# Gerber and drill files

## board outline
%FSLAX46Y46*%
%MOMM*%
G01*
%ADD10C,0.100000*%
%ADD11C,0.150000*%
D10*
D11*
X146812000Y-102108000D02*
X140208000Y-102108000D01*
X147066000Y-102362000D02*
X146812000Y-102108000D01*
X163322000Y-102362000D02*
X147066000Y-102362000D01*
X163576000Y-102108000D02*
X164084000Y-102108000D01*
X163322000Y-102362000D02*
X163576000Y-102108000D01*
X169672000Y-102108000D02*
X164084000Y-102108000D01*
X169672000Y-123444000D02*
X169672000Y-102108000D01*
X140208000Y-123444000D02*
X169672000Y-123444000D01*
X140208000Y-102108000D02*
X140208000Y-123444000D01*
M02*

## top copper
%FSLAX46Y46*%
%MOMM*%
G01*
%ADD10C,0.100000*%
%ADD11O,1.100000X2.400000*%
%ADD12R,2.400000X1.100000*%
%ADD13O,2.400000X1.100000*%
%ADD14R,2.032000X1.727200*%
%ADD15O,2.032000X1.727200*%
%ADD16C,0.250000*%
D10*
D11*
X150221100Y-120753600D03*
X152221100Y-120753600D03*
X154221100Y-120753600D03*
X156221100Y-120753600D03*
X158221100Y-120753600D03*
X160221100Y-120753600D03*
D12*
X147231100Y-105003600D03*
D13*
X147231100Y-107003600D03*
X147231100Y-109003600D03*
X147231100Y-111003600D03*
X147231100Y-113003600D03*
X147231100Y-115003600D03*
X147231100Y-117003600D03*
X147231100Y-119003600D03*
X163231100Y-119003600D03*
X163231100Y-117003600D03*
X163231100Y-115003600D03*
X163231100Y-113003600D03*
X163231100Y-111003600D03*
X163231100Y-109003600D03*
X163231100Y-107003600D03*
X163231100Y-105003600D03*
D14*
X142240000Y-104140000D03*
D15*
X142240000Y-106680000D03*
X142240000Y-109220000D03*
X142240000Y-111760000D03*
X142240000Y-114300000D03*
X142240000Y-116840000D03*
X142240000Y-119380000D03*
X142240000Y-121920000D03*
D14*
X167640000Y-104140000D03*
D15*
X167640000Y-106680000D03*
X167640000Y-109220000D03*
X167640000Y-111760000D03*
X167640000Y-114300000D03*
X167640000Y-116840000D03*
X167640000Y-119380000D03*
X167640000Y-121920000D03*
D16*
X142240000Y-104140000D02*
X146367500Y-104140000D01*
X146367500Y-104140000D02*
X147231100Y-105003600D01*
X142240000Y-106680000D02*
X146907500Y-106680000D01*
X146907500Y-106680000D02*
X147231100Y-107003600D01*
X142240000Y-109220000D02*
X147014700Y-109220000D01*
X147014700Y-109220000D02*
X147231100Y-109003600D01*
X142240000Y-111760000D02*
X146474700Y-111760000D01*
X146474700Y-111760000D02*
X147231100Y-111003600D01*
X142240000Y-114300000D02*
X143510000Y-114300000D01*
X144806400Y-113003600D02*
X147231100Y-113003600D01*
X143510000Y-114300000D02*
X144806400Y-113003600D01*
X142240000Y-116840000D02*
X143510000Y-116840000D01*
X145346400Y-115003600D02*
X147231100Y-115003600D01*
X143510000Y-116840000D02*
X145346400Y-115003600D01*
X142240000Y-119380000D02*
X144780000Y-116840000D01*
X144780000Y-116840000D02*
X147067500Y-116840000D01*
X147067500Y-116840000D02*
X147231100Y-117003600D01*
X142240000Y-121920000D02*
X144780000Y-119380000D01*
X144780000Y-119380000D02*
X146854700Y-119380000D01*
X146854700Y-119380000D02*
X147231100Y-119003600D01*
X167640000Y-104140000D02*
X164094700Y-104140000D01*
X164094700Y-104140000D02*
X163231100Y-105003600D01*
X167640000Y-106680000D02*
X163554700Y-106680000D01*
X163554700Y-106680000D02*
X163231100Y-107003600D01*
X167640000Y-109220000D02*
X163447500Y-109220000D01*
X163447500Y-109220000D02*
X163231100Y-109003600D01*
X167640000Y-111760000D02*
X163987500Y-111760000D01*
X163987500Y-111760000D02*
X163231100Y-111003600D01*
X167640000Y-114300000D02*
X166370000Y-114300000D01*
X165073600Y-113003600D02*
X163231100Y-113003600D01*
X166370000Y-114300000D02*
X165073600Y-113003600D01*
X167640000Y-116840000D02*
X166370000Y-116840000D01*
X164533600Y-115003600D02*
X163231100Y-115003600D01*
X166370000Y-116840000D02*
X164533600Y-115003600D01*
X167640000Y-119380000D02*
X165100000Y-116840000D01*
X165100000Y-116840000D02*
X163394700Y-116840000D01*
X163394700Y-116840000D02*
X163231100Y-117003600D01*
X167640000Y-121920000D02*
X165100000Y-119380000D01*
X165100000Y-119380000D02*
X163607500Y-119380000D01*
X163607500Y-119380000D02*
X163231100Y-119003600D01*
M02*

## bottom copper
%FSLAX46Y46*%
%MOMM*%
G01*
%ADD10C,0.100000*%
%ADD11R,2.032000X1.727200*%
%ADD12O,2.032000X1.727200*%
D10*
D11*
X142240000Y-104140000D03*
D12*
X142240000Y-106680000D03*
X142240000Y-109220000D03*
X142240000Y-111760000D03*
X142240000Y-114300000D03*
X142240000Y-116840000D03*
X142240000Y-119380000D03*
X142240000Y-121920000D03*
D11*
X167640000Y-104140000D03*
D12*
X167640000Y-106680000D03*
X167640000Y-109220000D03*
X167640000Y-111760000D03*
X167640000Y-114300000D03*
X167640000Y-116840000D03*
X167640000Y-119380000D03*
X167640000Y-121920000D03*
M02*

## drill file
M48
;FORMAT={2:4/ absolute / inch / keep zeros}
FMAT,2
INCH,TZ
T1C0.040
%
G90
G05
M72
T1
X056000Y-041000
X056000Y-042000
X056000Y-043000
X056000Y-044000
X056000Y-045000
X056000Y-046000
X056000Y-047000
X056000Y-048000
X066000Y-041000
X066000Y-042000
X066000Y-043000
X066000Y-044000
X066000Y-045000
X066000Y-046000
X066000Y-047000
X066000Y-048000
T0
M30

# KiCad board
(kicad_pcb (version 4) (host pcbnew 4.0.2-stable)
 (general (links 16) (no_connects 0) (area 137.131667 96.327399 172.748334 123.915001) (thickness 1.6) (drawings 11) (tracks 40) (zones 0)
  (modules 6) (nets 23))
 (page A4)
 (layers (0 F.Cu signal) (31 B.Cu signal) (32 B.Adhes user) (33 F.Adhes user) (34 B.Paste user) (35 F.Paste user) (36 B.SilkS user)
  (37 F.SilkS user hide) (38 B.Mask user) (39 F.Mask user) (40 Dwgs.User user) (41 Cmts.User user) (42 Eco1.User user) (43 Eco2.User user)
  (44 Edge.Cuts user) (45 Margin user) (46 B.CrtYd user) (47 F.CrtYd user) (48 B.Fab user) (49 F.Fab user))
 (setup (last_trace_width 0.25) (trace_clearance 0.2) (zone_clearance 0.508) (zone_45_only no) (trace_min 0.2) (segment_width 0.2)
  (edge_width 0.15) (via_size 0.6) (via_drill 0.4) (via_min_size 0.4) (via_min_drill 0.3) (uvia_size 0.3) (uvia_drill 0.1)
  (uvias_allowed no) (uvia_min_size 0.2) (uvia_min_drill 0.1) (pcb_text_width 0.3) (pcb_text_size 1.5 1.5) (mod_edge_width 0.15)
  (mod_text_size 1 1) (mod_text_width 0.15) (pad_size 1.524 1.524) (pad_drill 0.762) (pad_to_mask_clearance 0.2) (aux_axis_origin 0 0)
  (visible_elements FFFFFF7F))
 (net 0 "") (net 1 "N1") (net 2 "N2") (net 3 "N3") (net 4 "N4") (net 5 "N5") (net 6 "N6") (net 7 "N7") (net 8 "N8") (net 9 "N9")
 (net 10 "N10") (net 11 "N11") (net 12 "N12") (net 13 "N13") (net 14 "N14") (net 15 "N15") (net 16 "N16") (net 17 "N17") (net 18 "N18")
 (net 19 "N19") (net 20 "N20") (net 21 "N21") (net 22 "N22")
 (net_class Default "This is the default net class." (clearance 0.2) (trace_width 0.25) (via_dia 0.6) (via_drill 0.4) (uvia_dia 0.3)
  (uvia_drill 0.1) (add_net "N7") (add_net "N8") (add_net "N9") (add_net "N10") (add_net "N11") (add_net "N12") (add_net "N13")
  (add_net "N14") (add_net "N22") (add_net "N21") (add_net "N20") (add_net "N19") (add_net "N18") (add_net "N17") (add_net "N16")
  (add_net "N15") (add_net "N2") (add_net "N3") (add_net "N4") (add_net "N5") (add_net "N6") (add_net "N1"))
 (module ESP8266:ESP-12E (layer F.Cu) (at 147.2311 105.0036)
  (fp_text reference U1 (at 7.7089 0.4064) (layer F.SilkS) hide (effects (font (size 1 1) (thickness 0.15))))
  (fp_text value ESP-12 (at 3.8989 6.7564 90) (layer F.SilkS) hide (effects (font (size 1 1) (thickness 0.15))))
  (pad 9 smd oval (at 2.99 15.75 90) (size 2.4 1.1) (layers F.Cu F.Paste F.Mask) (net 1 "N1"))
  (pad 10 smd oval (at 4.99 15.75 90) (size 2.4 1.1) (layers F.Cu F.Paste F.Mask) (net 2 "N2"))
  (pad 11 smd oval (at 6.99 15.75 90) (size 2.4 1.1) (layers F.Cu F.Paste F.Mask) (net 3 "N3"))
  (pad 12 smd oval (at 8.99 15.75 90) (size 2.4 1.1) (layers F.Cu F.Paste F.Mask) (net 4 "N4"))
  (pad 13 smd oval (at 10.99 15.75 90) (size 2.4 1.1) (layers F.Cu F.Paste F.Mask) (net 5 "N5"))
  (pad 14 smd oval (at 12.99 15.75 90) (size 2.4 1.1) (layers F.Cu F.Paste F.Mask) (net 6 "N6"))
  (pad 1 smd rect (at 0 0) (size 2.4 1.1) (layers F.Cu F.Paste F.Mask) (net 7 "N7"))
  (pad 2 smd oval (at 0 2) (size 2.4 1.1) (layers F.Cu F.Paste F.Mask) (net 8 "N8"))
  (pad 3 smd oval (at 0 4) (size 2.4 1.1) (layers F.Cu F.Paste F.Mask) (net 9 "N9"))
  (pad 4 smd oval (at 0 6) (size 2.4 1.1) (layers F.Cu F.Paste F.Mask) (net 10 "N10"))
  (pad 5 smd oval (at 0 8) (size 2.4 1.1) (layers F.Cu F.Paste F.Mask) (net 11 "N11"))
  (pad 6 smd oval (at 0 10) (size 2.4 1.1) (layers F.Cu F.Paste F.Mask) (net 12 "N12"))
  (pad 7 smd oval (at 0 12) (size 2.4 1.1) (layers F.Cu F.Paste F.Mask) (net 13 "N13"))
  (pad 8 smd oval (at 0 14) (size 2.4 1.1) (layers F.Cu F.Paste F.Mask) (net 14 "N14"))
  (pad 15 smd oval (at 16 14) (size 2.4 1.1) (layers F.Cu F.Paste F.Mask) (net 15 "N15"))
  (pad 16 smd oval (at 16 12) (size 2.4 1.1) (layers F.Cu F.Paste F.Mask) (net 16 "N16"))
  (pad 17 smd oval (at 16 10) (size 2.4 1.1) (layers F.Cu F.Paste F.Mask) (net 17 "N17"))
  (pad 18 smd oval (at 16 8) (size 2.4 1.1) (layers F.Cu F.Paste F.Mask) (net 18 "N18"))
  (pad 19 smd oval (at 16 6) (size 2.4 1.1) (layers F.Cu F.Paste F.Mask) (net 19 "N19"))
  (pad 20 smd oval (at 16 4) (size 2.4 1.1) (layers F.Cu F.Paste F.Mask) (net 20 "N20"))
  (pad 21 smd oval (at 16 2) (size 2.4 1.1) (layers F.Cu F.Paste F.Mask) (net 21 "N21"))
  (pad 22 smd oval (at 16 0) (size 2.4 1.1) (layers F.Cu F.Paste F.Mask) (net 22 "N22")))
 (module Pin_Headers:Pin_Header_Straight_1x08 (layer F.Cu) (at 142.24 104.14)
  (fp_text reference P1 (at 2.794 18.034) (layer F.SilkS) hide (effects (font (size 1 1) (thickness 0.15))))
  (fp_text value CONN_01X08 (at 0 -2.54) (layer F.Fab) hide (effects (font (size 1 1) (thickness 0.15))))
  (pad 1 thru_hole rect (at 0 0) (size 2.032 1.7272) (drill 1.016) (layers *.Cu *.Mask F.SilkS) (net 7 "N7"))
  (pad 2 thru_hole oval (at 0 2.54) (size 2.032 1.7272) (drill 1.016) (layers *.Cu *.Mask F.SilkS) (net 8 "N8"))
  (pad 3 thru_hole oval (at 0 5.08) (size 2.032 1.7272) (drill 1.016) (layers *.Cu *.Mask F.SilkS) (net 9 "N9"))
  (pad 4 thru_hole oval (at 0 7.62) (size 2.032 1.7272) (drill 1.016) (layers *.Cu *.Mask F.SilkS) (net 10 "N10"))
  (pad 5 thru_hole oval (at 0 10.16) (size 2.032 1.7272) (drill 1.016) (layers *.Cu *.Mask F.SilkS) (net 11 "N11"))
  (pad 6 thru_hole oval (at 0 12.7) (size 2.032 1.7272) (drill 1.016) (layers *.Cu *.Mask F.SilkS) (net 12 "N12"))
  (pad 7 thru_hole oval (at 0 15.24) (size 2.032 1.7272) (drill 1.016) (layers *.Cu *.Mask F.SilkS) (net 13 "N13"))
  (pad 8 thru_hole oval (at 0 17.78) (size 2.032 1.7272) (drill 1.016) (layers *.Cu *.Mask F.SilkS) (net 14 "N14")))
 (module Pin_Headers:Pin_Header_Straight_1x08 (layer F.Cu) (at 167.64 104.14)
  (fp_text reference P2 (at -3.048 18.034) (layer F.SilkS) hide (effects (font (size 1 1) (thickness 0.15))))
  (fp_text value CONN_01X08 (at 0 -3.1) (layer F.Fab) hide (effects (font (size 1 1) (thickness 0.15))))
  (pad 1 thru_hole rect (at 0 0) (size 2.032 1.7272) (drill 1.016) (layers *.Cu *.Mask F.SilkS) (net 22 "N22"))
  (pad 2 thru_hole oval (at 0 2.54) (size 2.032 1.7272) (drill 1.016) (layers *.Cu *.Mask F.SilkS) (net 21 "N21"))
  (pad 3 thru_hole oval (at 0 5.08) (size 2.032 1.7272) (drill 1.016) (layers *.Cu *.Mask F.SilkS) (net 20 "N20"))
  (pad 4 thru_hole oval (at 0 7.62) (size 2.032 1.7272) (drill 1.016) (layers *.Cu *.Mask F.SilkS) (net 19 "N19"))
  (pad 5 thru_hole oval (at 0 10.16) (size 2.032 1.7272) (drill 1.016) (layers *.Cu *.Mask F.SilkS) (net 18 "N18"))
  (pad 6 thru_hole oval (at 0 12.7) (size 2.032 1.7272) (drill 1.016) (layers *.Cu *.Mask F.SilkS) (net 17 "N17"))
  (pad 7 thru_hole oval (at 0 15.24) (size 2.032 1.7272) (drill 1.016) (layers *.Cu *.Mask F.SilkS) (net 16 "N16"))
  (pad 8 thru_hole oval (at 0 17.78) (size 2.032 1.7272) (drill 1.016) (layers *.Cu *.Mask F.SilkS) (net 15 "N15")))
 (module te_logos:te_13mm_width (layer F.Cu) (at 159.258 111.506 90)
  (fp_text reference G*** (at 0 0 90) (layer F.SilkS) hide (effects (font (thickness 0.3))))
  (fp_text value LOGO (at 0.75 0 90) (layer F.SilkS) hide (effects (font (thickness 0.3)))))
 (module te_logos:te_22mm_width (layer B.Cu) (at 154.94 117.094 180)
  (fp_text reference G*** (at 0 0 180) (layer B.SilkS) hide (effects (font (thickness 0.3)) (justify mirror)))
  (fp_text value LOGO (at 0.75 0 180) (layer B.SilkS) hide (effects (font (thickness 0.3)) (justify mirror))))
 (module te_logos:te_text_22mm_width (layer B.Cu) (at 154.94 120.904 180)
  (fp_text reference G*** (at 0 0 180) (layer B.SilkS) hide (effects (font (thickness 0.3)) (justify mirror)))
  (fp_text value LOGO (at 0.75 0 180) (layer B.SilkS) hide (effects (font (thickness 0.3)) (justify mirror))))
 (gr_line (start 146.812 102.108) (end 140.208 102.108) (angle 90) (layer Edge.Cuts) (width 0.15))
 (gr_line (start 147.066 102.362) (end 146.812 102.108) (angle 90) (layer Edge.Cuts) (width 0.15))
 (gr_line (start 163.322 102.362) (end 147.066 102.362) (angle 90) (layer Edge.Cuts) (width 0.15))
 (gr_line (start 163.576 102.108) (end 164.084 102.108) (angle 90) (layer Edge.Cuts) (width 0.15))
 (gr_line (start 163.322 102.362) (end 163.576 102.108) (angle 90) (layer Edge.Cuts) (width 0.15))
 (gr_line (start 169.672 102.108) (end 164.084 102.108) (angle 90) (layer Edge.Cuts) (width 0.15))
 (gr_line (start 169.672 123.444) (end 169.672 102.108) (angle 90) (layer Edge.Cuts) (width 0.15))
 (gr_line (start 140.208 123.444) (end 169.672 123.444) (angle 90) (layer Edge.Cuts) (width 0.15))
 (gr_line (start 140.208 102.108) (end 140.208 123.444) (angle 90) (layer Edge.Cuts) (width 0.15))
 (segment (start 142.24 104.14) (end 146.3675 104.14) (width 0.25) (layer F.Cu) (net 7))
 (segment (start 146.3675 104.14) (end 147.2311 105.0036) (width 0.25) (layer F.Cu) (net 7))
 (segment (start 142.24 106.68) (end 146.9075 106.68) (width 0.25) (layer F.Cu) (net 8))
 (segment (start 146.9075 106.68) (end 147.2311 107.0036) (width 0.25) (layer F.Cu) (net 8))
 (segment (start 142.24 109.22) (end 147.0147 109.22) (width 0.25) (layer F.Cu) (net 9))
 (segment (start 147.0147 109.22) (end 147.2311 109.0036) (width 0.25) (layer F.Cu) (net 9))
 (segment (start 142.24 111.76) (end 146.4747 111.76) (width 0.25) (layer F.Cu) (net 10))
 (segment (start 146.4747 111.76) (end 147.2311 111.0036) (width 0.25) (layer F.Cu) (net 10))
 (segment (start 142.24 114.3) (end 143.51 114.3) (width 0.25) (layer F.Cu) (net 11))
 (segment (start 144.8064 113.0036) (end 147.2311 113.0036) (width 0.25) (layer F.Cu) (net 11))
 (segment (start 143.51 114.3) (end 144.8064 113.0036) (width 0.25) (layer F.Cu) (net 11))
 (segment (start 142.24 116.84) (end 143.51 116.84) (width 0.25) (layer F.Cu) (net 12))
 (segment (start 145.3464 115.0036) (end 147.2311 115.0036) (width 0.25) (layer F.Cu) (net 12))
 (segment (start 143.51 116.84) (end 145.3464 115.0036) (width 0.25) (layer F.Cu) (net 12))
 (segment (start 142.24 119.38) (end 144.78 116.84) (width 0.25) (layer F.Cu) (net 13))
 (segment (start 144.78 116.84) (end 147.0675 116.84) (width 0.25) (layer F.Cu) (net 13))
 (segment (start 147.0675 116.84) (end 147.2311 117.0036) (width 0.25) (layer F.Cu) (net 13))
 (segment (start 142.24 121.92) (end 144.78 119.38) (width 0.25) (layer F.Cu) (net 14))
 (segment (start 144.78 119.38) (end 146.8547 119.38) (width 0.25) (layer F.Cu) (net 14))
 (segment (start 146.8547 119.38) (end 147.2311 119.0036) (width 0.25) (layer F.Cu) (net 14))
 (segment (start 167.64 104.14) (end 164.0947 104.14) (width 0.25) (layer F.Cu) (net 22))
 (segment (start 164.0947 104.14) (end 163.2311 105.0036) (width 0.25) (layer F.Cu) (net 22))
 (segment (start 167.64 106.68) (end 163.5547 106.68) (width 0.25) (layer F.Cu) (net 21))
 (segment (start 163.5547 106.68) (end 163.2311 107.0036) (width 0.25) (layer F.Cu) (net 21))
 (segment (start 167.64 109.22) (end 163.4475 109.22) (width 0.25) (layer F.Cu) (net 20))
 (segment (start 163.4475 109.22) (end 163.2311 109.0036) (width 0.25) (layer F.Cu) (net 20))
 (segment (start 167.64 111.76) (end 163.9875 111.76) (width 0.25) (layer F.Cu) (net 19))
 (segment (start 163.9875 111.76) (end 163.2311 111.0036) (width 0.25) (layer F.Cu) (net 19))
 (segment (start 167.64 114.3) (end 166.37 114.3) (width 0.25) (layer F.Cu) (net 18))
 (segment (start 165.0736 113.0036) (end 163.2311 113.0036) (width 0.25) (layer F.Cu) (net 18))
 (segment (start 166.37 114.3) (end 165.0736 113.0036) (width 0.25) (layer F.Cu) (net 18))
 (segment (start 167.64 116.84) (end 166.37 116.84) (width 0.25) (layer F.Cu) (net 17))
 (segment (start 164.5336 115.0036) (end 163.2311 115.0036) (width 0.25) (layer F.Cu) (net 17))
 (segment (start 166.37 116.84) (end 164.5336 115.0036) (width 0.25) (layer F.Cu) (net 17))
 (segment (start 167.64 119.38) (end 165.1 116.84) (width 0.25) (layer F.Cu) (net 16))
 (segment (start 165.1 116.84) (end 163.3947 116.84) (width 0.25) (layer F.Cu) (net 16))
 (segment (start 163.3947 116.84) (end 163.2311 117.0036) (width 0.25) (layer F.Cu) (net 16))
 (segment (start 167.64 121.92) (end 165.1 119.38) (width 0.25) (layer F.Cu) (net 15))
 (segment (start 165.1 119.38) (end 163.6075 119.38) (width 0.25) (layer F.Cu) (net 15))
 (segment (start 163.6075 119.38) (end 163.2311 119.0036) (width 0.25) (layer F.Cu) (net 15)))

